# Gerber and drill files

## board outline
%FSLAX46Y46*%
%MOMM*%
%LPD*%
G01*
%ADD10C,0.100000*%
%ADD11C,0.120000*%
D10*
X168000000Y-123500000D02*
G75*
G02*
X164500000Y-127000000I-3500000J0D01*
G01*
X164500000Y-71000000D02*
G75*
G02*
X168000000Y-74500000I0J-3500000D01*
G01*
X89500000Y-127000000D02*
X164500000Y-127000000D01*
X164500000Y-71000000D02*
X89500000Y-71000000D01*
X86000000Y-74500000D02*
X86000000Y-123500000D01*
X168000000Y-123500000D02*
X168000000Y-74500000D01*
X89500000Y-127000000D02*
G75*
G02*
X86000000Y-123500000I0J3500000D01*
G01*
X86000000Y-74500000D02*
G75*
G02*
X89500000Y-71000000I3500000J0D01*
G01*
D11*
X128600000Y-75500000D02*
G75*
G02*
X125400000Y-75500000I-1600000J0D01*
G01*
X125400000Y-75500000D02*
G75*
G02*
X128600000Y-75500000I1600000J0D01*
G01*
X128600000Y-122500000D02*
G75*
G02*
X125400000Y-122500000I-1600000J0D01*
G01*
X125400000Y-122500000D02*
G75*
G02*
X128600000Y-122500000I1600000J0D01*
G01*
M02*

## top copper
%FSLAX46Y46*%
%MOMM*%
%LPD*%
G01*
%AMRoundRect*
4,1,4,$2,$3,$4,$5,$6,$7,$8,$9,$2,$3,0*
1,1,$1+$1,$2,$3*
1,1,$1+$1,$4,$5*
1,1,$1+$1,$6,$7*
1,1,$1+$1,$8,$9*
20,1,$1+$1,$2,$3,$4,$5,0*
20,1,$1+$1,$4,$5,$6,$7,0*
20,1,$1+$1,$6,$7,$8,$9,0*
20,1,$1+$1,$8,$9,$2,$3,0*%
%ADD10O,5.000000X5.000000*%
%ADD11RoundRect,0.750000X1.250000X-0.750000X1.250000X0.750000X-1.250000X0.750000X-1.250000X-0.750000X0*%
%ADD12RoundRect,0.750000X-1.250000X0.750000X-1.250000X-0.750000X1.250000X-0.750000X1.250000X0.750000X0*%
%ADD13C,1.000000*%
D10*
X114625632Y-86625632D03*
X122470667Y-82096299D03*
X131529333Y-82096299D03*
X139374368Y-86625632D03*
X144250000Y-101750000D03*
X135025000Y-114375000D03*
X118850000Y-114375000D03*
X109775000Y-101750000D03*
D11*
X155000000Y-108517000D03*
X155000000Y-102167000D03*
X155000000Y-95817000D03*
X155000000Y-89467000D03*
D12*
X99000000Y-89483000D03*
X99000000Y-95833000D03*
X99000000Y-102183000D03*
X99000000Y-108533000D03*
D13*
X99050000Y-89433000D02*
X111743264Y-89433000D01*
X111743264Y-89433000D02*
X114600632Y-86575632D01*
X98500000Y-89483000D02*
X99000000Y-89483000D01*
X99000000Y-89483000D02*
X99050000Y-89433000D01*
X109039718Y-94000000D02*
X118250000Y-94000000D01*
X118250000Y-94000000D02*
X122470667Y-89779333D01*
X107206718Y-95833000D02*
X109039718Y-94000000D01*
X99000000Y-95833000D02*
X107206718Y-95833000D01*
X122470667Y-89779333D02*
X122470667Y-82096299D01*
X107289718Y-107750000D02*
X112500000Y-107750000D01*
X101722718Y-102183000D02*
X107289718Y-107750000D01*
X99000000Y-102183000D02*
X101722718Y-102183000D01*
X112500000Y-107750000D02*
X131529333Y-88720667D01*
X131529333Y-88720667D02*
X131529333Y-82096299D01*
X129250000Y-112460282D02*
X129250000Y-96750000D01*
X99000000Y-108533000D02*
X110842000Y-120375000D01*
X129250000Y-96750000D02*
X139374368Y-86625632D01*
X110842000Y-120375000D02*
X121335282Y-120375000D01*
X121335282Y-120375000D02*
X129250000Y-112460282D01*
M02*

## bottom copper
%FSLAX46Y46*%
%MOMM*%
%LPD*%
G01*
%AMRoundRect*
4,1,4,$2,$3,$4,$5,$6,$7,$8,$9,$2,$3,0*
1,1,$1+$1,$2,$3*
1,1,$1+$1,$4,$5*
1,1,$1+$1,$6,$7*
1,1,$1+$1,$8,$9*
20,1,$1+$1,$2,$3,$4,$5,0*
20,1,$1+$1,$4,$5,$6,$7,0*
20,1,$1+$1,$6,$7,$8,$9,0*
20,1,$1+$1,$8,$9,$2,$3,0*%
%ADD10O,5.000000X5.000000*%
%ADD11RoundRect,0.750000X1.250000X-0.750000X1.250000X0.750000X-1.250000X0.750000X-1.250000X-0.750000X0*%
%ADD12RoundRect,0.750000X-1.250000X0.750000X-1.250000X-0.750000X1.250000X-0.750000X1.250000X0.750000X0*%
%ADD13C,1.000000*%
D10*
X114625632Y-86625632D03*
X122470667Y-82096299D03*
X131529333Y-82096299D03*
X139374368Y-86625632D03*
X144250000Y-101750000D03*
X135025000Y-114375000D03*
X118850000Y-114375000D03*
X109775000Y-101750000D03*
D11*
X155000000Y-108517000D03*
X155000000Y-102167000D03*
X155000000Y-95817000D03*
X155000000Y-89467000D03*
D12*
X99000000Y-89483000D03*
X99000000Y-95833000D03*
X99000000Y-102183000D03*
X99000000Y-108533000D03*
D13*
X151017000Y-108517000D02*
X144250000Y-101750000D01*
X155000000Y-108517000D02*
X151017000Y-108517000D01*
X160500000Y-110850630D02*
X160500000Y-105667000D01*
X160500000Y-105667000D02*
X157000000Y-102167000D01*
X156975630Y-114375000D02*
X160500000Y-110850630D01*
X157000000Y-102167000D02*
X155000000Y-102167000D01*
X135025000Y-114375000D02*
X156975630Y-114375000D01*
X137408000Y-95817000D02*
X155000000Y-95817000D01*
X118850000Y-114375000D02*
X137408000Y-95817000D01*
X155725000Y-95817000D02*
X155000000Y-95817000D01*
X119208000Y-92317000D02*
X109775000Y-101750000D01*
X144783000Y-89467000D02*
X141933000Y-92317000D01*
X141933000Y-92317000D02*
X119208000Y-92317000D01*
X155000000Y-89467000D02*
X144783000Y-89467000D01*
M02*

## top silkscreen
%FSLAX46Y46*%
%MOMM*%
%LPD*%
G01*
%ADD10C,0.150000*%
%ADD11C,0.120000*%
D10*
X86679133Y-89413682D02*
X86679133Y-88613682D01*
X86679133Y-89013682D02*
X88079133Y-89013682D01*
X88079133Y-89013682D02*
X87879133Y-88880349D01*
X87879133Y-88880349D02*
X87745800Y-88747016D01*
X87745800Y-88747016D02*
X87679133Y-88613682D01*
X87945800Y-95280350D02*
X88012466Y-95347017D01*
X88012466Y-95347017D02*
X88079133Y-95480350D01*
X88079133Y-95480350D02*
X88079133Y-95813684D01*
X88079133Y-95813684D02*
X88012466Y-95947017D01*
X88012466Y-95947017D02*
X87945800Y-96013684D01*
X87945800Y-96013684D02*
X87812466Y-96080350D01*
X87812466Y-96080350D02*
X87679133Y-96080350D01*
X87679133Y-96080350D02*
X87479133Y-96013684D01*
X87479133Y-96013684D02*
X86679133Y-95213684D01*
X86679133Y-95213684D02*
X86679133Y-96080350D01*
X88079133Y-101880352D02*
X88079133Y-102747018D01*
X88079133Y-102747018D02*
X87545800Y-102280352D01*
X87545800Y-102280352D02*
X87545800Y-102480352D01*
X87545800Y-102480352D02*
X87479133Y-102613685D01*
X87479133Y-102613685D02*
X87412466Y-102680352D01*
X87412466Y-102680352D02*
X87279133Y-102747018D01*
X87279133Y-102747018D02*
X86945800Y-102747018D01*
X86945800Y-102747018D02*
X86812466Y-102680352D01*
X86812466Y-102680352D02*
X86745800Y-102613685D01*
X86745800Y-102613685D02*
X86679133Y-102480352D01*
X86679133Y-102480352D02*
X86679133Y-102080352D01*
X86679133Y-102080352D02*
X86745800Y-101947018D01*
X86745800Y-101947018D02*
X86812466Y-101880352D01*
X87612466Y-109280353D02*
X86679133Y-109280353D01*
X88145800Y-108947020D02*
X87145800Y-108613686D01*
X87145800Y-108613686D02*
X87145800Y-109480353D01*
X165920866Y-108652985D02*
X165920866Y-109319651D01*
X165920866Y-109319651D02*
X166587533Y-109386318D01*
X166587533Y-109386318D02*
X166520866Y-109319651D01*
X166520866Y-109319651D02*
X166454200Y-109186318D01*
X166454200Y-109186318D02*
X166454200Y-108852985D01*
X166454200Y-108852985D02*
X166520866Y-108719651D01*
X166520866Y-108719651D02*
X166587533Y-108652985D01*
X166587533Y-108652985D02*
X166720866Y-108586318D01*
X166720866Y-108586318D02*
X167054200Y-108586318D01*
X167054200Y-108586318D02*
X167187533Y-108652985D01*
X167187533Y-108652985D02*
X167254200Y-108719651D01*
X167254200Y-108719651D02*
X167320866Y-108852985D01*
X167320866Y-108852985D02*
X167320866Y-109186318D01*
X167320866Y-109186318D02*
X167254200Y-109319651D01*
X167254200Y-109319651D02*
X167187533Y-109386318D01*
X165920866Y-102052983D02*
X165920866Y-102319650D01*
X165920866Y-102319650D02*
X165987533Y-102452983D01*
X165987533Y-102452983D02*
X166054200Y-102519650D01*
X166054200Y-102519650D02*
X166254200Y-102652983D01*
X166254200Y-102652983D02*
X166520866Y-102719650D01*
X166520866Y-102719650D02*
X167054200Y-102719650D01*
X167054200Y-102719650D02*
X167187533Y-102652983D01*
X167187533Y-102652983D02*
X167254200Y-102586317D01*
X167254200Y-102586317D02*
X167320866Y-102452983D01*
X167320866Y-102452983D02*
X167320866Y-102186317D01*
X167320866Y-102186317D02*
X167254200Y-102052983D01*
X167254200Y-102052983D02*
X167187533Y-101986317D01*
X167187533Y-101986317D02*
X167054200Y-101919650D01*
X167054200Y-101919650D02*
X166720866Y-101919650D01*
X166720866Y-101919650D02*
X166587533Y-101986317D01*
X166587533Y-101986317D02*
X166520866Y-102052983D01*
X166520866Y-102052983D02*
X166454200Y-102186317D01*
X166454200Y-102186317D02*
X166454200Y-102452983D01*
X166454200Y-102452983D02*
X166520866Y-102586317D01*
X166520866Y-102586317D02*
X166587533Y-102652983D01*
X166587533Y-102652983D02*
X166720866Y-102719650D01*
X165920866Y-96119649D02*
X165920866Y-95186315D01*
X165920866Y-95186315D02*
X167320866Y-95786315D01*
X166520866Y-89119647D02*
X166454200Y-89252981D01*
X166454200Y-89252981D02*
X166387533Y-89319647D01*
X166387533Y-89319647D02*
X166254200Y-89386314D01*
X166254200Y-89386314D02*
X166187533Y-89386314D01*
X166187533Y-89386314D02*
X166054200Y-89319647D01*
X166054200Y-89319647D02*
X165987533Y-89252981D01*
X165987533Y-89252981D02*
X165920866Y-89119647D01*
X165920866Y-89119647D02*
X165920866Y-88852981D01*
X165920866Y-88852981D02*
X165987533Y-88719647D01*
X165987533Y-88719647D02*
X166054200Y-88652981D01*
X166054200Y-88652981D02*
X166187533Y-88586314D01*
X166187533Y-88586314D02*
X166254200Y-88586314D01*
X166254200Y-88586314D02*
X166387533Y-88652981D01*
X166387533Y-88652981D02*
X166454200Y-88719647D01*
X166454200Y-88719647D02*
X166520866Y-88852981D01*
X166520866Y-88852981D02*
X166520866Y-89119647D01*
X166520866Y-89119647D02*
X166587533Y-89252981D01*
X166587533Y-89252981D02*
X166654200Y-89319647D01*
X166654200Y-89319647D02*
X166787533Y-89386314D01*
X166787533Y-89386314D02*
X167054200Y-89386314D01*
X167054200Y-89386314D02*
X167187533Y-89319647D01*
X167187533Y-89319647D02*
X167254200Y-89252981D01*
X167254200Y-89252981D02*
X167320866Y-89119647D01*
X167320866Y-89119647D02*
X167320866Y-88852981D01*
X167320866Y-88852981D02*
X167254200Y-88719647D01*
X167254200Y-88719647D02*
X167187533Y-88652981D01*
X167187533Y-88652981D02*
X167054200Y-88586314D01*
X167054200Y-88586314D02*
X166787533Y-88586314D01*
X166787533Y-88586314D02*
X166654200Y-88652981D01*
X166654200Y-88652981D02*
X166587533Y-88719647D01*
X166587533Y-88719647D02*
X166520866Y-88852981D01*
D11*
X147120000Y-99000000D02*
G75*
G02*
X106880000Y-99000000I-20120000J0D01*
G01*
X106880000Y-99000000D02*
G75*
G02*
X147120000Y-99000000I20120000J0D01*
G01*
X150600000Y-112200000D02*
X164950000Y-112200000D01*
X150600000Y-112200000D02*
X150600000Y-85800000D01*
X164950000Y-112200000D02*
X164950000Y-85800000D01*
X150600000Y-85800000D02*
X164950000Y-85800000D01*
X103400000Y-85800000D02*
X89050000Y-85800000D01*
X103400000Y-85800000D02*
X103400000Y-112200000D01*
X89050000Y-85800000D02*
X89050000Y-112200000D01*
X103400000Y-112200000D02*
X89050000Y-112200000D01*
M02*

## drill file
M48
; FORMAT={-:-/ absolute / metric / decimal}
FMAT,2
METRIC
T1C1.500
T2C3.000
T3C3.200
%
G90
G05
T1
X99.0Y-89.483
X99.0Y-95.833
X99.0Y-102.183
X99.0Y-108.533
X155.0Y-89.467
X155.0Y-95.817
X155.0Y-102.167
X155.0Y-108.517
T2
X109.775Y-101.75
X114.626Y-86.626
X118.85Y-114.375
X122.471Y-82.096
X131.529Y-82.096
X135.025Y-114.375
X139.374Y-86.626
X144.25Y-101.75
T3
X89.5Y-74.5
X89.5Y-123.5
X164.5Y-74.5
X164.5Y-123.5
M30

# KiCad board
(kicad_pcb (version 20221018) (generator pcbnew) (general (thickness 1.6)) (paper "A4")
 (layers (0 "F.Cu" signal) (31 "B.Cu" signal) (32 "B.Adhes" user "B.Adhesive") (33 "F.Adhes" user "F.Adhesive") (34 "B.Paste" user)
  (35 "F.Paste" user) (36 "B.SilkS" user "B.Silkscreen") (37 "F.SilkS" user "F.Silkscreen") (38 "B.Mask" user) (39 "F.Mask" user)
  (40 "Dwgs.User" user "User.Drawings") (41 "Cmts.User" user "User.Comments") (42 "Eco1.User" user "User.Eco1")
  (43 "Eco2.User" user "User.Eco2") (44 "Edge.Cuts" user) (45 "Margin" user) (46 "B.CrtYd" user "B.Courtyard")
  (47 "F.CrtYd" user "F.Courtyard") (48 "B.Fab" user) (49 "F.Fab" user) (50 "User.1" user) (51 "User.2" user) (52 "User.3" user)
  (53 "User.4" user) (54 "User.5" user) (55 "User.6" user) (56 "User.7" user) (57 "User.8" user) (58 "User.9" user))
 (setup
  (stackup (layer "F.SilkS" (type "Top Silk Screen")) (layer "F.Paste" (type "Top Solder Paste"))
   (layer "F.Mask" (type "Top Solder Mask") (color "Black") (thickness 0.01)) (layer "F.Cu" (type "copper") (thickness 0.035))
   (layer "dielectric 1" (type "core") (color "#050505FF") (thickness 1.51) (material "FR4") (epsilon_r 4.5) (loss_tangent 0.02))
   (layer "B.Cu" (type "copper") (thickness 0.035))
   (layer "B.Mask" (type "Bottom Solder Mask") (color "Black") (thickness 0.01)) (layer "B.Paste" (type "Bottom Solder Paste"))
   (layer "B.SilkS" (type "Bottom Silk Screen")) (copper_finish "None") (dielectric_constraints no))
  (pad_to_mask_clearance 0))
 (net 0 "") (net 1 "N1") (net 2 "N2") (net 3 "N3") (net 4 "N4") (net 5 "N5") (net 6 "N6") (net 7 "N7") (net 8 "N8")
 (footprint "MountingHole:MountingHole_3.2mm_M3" (layer "F.Cu") (at 89.5 123.5)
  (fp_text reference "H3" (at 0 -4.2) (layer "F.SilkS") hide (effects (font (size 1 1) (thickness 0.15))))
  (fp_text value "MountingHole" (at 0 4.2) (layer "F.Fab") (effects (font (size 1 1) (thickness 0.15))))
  (pad "" np_thru_hole circle (at 0 0) (size 3.2 3.2) (drill 3.2) (layers "*.Cu" "*.Mask")))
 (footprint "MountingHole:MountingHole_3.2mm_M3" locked (layer "F.Cu") (at 164.5 123.5)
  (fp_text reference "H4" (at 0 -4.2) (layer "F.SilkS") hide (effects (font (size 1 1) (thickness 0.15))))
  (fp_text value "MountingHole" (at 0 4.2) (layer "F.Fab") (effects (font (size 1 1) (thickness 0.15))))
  (pad "" np_thru_hole circle locked (at 0 0) (size 3.2 3.2) (drill 3.2) (layers "*.Cu" "*.Mask")))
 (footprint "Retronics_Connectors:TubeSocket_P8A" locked (layer "F.Cu") (at 127 99)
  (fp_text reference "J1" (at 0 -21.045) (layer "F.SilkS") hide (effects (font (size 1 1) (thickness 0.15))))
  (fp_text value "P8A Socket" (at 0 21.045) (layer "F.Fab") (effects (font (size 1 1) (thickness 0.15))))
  (fp_circle (center 0 0) (end 0 20.12) (stroke (width 0.12) (type default)) (fill none) (layer "F.SilkS"))
  (fp_circle (center 0 -23.5) (end 1.6 -23.5) (stroke (width 0.12) (type default)) (fill none) (layer "Edge.Cuts"))
  (fp_circle (center 0 23.5) (end 1.6 23.5) (stroke (width 0.12) (type default)) (fill none) (layer "Edge.Cuts"))
  (pad "1" thru_hole oval locked (at -12.374368 -12.374368) (size 5 5) (drill 3) (layers "*.Cu" "*.Mask") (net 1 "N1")
   (thermal_bridge_angle 45))
  (pad "2" thru_hole oval locked (at -4.529333 -16.903701) (size 5 5) (drill 3) (layers "*.Cu" "*.Mask") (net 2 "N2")
   (thermal_bridge_angle 45))
  (pad "3" thru_hole oval locked (at 4.529333 -16.903701) (size 5 5) (drill 3) (layers "*.Cu" "*.Mask") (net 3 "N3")
   (thermal_bridge_angle 45))
  (pad "4" thru_hole oval locked (at 12.374368 -12.374368) (size 5 5) (drill 3) (layers "*.Cu" "*.Mask") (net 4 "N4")
   (thermal_bridge_angle 45))
  (pad "5" thru_hole oval locked (at 17.25 2.75) (size 5 5) (drill 3) (layers "*.Cu" "*.Mask") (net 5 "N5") (thermal_bridge_angle 45))
  (pad "6" thru_hole oval locked (at 8.025 15.375) (size 5 5) (drill 3) (layers "*.Cu" "*.Mask") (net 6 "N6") (thermal_bridge_angle 45))
  (pad "7" thru_hole oval locked (at -8.15 15.375) (size 5 5) (drill 3) (layers "*.Cu" "*.Mask") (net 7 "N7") (thermal_bridge_angle 45))
  (pad "8" thru_hole oval locked (at -17.225 2.75) (size 5 5) (drill 3) (layers "*.Cu" "*.Mask") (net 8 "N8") (thermal_bridge_angle 45)))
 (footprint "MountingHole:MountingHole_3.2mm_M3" (layer "F.Cu") (at 89.5 74.5)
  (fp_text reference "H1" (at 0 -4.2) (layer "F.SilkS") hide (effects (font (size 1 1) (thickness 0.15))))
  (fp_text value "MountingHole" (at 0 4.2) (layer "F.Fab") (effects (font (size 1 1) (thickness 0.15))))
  (pad "" np_thru_hole circle (at 0 0) (size 3.2 3.2) (drill 3.2) (layers "*.Cu" "*.Mask")))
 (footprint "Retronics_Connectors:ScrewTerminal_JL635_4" (layer "F.Cu") (at 155 108.517 90)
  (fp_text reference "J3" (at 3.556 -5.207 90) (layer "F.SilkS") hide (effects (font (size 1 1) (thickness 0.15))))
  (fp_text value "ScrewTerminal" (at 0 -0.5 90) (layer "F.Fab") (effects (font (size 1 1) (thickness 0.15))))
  (fp_line (start -3.683 -4.4) (end -3.683 9.95) (stroke (width 0.12) (type solid)) (layer "F.SilkS"))
  (fp_line (start -3.683 -4.4) (end 22.717 -4.4) (stroke (width 0.12) (type solid)) (layer "F.SilkS"))
  (fp_line (start -3.683 9.95) (end 22.717 9.95) (stroke (width 0.12) (type solid)) (layer "F.SilkS"))
  (fp_line (start 22.717 -4.4) (end 22.717 9.95) (stroke (width 0.12) (type solid)) (layer "F.SilkS"))
  (pad "1" thru_hole roundrect (at 0 0 90) (size 3 4) (drill 1.5) (layers "*.Cu" "*.Mask") (roundrect_rratio 0.25) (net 5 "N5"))
  (pad "2" thru_hole roundrect (at 6.35 0 90) (size 3 4) (drill 1.5) (layers "*.Cu" "*.Mask") (roundrect_rratio 0.25) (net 6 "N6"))
  (pad "3" thru_hole roundrect (at 12.7 0 90) (size 3 4) (drill 1.5) (layers "*.Cu" "*.Mask") (roundrect_rratio 0.25) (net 7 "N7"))
  (pad "4" thru_hole roundrect (at 19.05 0 90) (size 3 4) (drill 1.5) (layers "*.Cu" "*.Mask") (roundrect_rratio 0.25) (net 8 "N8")))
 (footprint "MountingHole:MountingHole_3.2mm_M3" (layer "F.Cu") (at 164.5 74.5)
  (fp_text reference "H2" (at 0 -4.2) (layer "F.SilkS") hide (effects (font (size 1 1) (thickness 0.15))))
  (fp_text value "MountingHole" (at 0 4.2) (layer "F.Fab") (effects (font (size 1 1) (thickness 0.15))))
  (pad "" np_thru_hole circle (at 0 0) (size 3.2 3.2) (drill 3.2) (layers "*.Cu" "*.Mask")))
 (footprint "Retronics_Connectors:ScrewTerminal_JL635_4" (layer "F.Cu") (at 99 89.483 -90)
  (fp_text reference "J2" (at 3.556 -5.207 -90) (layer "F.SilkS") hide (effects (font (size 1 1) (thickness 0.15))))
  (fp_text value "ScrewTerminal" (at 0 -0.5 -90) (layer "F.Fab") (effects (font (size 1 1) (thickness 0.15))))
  (fp_line (start -3.683 -4.4) (end -3.683 9.95) (stroke (width 0.12) (type solid)) (layer "F.SilkS"))
  (fp_line (start -3.683 -4.4) (end 22.717 -4.4) (stroke (width 0.12) (type solid)) (layer "F.SilkS"))
  (fp_line (start -3.683 9.95) (end 22.717 9.95) (stroke (width 0.12) (type solid)) (layer "F.SilkS"))
  (fp_line (start 22.717 -4.4) (end 22.717 9.95) (stroke (width 0.12) (type solid)) (layer "F.SilkS"))
  (pad "1" thru_hole roundrect (at 0 0 270) (size 3 4) (drill 1.5) (layers "*.Cu" "*.Mask") (roundrect_rratio 0.25) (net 1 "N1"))
  (pad "2" thru_hole roundrect (at 6.35 0 270) (size 3 4) (drill 1.5) (layers "*.Cu" "*.Mask") (roundrect_rratio 0.25) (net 2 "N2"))
  (pad "3" thru_hole roundrect (at 12.7 0 270) (size 3 4) (drill 1.5) (layers "*.Cu" "*.Mask") (roundrect_rratio 0.25) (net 3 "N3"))
  (pad "4" thru_hole roundrect (at 19.05 0 270) (size 3 4) (drill 1.5) (layers "*.Cu" "*.Mask") (roundrect_rratio 0.25) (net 4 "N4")))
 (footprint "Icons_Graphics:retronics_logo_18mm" (layer "B.Cu") (at 126.995721 95.5 180)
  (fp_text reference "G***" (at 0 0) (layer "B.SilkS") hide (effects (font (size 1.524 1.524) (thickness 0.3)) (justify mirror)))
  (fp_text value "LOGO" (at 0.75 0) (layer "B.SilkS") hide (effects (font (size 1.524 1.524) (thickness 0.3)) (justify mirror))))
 (gr_arc (start 168 123.5) (mid 166.974874 125.974874) (end 164.5 127) (stroke (width 0.1) (type default)) (layer "Edge.Cuts"))
 (gr_arc (start 164.5 71) (mid 166.974874 72.025126) (end 168 74.5) (stroke (width 0.1) (type default)) (layer "Edge.Cuts"))
 (gr_line (start 89.5 127) (end 164.5 127) (stroke (width 0.1) (type default)) (layer "Edge.Cuts"))
 (gr_line (start 164.5 71) (end 89.5 71) (stroke (width 0.1) (type default)) (layer "Edge.Cuts"))
 (gr_line (start 86 74.5) (end 86 123.5) (stroke (width 0.1) (type default)) (layer "Edge.Cuts"))
 (gr_line (start 168 123.5) (end 168 74.5) (stroke (width 0.1) (type default)) (layer "Edge.Cuts"))
 (gr_arc (start 89.5 127) (mid 87.025126 125.974874) (end 86 123.5) (stroke (width 0.1) (type default)) (layer "Edge.Cuts"))
 (gr_arc (start 86 74.5) (mid 87.025126 72.025126) (end 89.5 71) (stroke (width 0.1) (type default)) (layer "Edge.Cuts"))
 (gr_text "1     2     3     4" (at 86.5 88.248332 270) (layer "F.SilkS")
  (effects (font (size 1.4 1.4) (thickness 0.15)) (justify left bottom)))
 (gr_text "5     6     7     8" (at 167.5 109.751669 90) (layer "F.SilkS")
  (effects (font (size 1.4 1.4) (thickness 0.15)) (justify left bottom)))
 (segment (start 99.05 89.433) (end 111.743264 89.433) (width 1) (layer "F.Cu") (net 1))
 (segment (start 111.743264 89.433) (end 114.600632 86.575632) (width 1) (layer "F.Cu") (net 1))
 (segment (start 98.5 89.483) (end 99 89.483) (width 1) (layer "F.Cu") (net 1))
 (segment (start 99 89.483) (end 99.05 89.433) (width 1) (layer "F.Cu") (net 1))
 (segment (start 109.039718 94) (end 118.25 94) (width 1) (layer "F.Cu") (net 2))
 (segment (start 118.25 94) (end 122.470667 89.779333) (width 1) (layer "F.Cu") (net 2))
 (segment (start 107.206718 95.833) (end 109.039718 94) (width 1) (layer "F.Cu") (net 2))
 (segment (start 99 95.833) (end 107.206718 95.833) (width 1) (layer "F.Cu") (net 2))
 (segment (start 122.470667 89.779333) (end 122.470667 82.096299) (width 1) (layer "F.Cu") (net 2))
 (segment (start 107.289718 107.75) (end 112.5 107.75) (width 1) (layer "F.Cu") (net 3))
 (segment (start 101.722718 102.183) (end 107.289718 107.75) (width 1) (layer "F.Cu") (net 3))
 (segment (start 99 102.183) (end 101.722718 102.183) (width 1) (layer "F.Cu") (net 3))
 (segment (start 112.5 107.75) (end 131.529333 88.720667) (width 1) (layer "F.Cu") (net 3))
 (segment (start 131.529333 88.720667) (end 131.529333 82.096299) (width 1) (layer "F.Cu") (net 3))
 (segment (start 129.25 112.460282) (end 129.25 96.75) (width 1) (layer "F.Cu") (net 4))
 (segment (start 99 108.533) (end 110.842 120.375) (width 1) (layer "F.Cu") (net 4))
 (segment (start 129.25 96.75) (end 139.374368 86.625632) (width 1) (layer "F.Cu") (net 4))
 (segment (start 110.842 120.375) (end 121.335282 120.375) (width 1) (layer "F.Cu") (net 4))
 (segment (start 121.335282 120.375) (end 129.25 112.460282) (width 1) (layer "F.Cu") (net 4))
 (segment (start 151.017 108.517) (end 144.25 101.75) (width 1) (layer "B.Cu") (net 5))
 (segment (start 155 108.517) (end 151.017 108.517) (width 1) (layer "B.Cu") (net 5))
 (segment (start 160.5 110.85063) (end 160.5 105.667) (width 1) (layer "B.Cu") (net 6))
 (segment (start 160.5 105.667) (end 157 102.167) (width 1) (layer "B.Cu") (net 6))
 (segment (start 156.97563 114.375) (end 160.5 110.85063) (width 1) (layer "B.Cu") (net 6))
 (segment (start 157 102.167) (end 155 102.167) (width 1) (layer "B.Cu") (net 6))
 (segment (start 135.025 114.375) (end 156.97563 114.375) (width 1) (layer "B.Cu") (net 6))
 (segment (start 137.408 95.817) (end 155 95.817) (width 1) (layer "B.Cu") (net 7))
 (segment (start 118.85 114.375) (end 137.408 95.817) (width 1) (layer "B.Cu") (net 7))
 (segment (start 155.725 95.817) (end 155 95.817) (width 1) (layer "B.Cu") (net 7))
 (segment (start 119.208 92.317) (end 109.775 101.75) (width 1) (layer "B.Cu") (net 8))
 (segment (start 144.783 89.467) (end 141.933 92.317) (width 1) (layer "B.Cu") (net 8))
 (segment (start 141.933 92.317) (end 119.208 92.317) (width 1) (layer "B.Cu") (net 8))
 (segment (start 155 89.467) (end 144.783 89.467) (width 1) (layer "B.Cu") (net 8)))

